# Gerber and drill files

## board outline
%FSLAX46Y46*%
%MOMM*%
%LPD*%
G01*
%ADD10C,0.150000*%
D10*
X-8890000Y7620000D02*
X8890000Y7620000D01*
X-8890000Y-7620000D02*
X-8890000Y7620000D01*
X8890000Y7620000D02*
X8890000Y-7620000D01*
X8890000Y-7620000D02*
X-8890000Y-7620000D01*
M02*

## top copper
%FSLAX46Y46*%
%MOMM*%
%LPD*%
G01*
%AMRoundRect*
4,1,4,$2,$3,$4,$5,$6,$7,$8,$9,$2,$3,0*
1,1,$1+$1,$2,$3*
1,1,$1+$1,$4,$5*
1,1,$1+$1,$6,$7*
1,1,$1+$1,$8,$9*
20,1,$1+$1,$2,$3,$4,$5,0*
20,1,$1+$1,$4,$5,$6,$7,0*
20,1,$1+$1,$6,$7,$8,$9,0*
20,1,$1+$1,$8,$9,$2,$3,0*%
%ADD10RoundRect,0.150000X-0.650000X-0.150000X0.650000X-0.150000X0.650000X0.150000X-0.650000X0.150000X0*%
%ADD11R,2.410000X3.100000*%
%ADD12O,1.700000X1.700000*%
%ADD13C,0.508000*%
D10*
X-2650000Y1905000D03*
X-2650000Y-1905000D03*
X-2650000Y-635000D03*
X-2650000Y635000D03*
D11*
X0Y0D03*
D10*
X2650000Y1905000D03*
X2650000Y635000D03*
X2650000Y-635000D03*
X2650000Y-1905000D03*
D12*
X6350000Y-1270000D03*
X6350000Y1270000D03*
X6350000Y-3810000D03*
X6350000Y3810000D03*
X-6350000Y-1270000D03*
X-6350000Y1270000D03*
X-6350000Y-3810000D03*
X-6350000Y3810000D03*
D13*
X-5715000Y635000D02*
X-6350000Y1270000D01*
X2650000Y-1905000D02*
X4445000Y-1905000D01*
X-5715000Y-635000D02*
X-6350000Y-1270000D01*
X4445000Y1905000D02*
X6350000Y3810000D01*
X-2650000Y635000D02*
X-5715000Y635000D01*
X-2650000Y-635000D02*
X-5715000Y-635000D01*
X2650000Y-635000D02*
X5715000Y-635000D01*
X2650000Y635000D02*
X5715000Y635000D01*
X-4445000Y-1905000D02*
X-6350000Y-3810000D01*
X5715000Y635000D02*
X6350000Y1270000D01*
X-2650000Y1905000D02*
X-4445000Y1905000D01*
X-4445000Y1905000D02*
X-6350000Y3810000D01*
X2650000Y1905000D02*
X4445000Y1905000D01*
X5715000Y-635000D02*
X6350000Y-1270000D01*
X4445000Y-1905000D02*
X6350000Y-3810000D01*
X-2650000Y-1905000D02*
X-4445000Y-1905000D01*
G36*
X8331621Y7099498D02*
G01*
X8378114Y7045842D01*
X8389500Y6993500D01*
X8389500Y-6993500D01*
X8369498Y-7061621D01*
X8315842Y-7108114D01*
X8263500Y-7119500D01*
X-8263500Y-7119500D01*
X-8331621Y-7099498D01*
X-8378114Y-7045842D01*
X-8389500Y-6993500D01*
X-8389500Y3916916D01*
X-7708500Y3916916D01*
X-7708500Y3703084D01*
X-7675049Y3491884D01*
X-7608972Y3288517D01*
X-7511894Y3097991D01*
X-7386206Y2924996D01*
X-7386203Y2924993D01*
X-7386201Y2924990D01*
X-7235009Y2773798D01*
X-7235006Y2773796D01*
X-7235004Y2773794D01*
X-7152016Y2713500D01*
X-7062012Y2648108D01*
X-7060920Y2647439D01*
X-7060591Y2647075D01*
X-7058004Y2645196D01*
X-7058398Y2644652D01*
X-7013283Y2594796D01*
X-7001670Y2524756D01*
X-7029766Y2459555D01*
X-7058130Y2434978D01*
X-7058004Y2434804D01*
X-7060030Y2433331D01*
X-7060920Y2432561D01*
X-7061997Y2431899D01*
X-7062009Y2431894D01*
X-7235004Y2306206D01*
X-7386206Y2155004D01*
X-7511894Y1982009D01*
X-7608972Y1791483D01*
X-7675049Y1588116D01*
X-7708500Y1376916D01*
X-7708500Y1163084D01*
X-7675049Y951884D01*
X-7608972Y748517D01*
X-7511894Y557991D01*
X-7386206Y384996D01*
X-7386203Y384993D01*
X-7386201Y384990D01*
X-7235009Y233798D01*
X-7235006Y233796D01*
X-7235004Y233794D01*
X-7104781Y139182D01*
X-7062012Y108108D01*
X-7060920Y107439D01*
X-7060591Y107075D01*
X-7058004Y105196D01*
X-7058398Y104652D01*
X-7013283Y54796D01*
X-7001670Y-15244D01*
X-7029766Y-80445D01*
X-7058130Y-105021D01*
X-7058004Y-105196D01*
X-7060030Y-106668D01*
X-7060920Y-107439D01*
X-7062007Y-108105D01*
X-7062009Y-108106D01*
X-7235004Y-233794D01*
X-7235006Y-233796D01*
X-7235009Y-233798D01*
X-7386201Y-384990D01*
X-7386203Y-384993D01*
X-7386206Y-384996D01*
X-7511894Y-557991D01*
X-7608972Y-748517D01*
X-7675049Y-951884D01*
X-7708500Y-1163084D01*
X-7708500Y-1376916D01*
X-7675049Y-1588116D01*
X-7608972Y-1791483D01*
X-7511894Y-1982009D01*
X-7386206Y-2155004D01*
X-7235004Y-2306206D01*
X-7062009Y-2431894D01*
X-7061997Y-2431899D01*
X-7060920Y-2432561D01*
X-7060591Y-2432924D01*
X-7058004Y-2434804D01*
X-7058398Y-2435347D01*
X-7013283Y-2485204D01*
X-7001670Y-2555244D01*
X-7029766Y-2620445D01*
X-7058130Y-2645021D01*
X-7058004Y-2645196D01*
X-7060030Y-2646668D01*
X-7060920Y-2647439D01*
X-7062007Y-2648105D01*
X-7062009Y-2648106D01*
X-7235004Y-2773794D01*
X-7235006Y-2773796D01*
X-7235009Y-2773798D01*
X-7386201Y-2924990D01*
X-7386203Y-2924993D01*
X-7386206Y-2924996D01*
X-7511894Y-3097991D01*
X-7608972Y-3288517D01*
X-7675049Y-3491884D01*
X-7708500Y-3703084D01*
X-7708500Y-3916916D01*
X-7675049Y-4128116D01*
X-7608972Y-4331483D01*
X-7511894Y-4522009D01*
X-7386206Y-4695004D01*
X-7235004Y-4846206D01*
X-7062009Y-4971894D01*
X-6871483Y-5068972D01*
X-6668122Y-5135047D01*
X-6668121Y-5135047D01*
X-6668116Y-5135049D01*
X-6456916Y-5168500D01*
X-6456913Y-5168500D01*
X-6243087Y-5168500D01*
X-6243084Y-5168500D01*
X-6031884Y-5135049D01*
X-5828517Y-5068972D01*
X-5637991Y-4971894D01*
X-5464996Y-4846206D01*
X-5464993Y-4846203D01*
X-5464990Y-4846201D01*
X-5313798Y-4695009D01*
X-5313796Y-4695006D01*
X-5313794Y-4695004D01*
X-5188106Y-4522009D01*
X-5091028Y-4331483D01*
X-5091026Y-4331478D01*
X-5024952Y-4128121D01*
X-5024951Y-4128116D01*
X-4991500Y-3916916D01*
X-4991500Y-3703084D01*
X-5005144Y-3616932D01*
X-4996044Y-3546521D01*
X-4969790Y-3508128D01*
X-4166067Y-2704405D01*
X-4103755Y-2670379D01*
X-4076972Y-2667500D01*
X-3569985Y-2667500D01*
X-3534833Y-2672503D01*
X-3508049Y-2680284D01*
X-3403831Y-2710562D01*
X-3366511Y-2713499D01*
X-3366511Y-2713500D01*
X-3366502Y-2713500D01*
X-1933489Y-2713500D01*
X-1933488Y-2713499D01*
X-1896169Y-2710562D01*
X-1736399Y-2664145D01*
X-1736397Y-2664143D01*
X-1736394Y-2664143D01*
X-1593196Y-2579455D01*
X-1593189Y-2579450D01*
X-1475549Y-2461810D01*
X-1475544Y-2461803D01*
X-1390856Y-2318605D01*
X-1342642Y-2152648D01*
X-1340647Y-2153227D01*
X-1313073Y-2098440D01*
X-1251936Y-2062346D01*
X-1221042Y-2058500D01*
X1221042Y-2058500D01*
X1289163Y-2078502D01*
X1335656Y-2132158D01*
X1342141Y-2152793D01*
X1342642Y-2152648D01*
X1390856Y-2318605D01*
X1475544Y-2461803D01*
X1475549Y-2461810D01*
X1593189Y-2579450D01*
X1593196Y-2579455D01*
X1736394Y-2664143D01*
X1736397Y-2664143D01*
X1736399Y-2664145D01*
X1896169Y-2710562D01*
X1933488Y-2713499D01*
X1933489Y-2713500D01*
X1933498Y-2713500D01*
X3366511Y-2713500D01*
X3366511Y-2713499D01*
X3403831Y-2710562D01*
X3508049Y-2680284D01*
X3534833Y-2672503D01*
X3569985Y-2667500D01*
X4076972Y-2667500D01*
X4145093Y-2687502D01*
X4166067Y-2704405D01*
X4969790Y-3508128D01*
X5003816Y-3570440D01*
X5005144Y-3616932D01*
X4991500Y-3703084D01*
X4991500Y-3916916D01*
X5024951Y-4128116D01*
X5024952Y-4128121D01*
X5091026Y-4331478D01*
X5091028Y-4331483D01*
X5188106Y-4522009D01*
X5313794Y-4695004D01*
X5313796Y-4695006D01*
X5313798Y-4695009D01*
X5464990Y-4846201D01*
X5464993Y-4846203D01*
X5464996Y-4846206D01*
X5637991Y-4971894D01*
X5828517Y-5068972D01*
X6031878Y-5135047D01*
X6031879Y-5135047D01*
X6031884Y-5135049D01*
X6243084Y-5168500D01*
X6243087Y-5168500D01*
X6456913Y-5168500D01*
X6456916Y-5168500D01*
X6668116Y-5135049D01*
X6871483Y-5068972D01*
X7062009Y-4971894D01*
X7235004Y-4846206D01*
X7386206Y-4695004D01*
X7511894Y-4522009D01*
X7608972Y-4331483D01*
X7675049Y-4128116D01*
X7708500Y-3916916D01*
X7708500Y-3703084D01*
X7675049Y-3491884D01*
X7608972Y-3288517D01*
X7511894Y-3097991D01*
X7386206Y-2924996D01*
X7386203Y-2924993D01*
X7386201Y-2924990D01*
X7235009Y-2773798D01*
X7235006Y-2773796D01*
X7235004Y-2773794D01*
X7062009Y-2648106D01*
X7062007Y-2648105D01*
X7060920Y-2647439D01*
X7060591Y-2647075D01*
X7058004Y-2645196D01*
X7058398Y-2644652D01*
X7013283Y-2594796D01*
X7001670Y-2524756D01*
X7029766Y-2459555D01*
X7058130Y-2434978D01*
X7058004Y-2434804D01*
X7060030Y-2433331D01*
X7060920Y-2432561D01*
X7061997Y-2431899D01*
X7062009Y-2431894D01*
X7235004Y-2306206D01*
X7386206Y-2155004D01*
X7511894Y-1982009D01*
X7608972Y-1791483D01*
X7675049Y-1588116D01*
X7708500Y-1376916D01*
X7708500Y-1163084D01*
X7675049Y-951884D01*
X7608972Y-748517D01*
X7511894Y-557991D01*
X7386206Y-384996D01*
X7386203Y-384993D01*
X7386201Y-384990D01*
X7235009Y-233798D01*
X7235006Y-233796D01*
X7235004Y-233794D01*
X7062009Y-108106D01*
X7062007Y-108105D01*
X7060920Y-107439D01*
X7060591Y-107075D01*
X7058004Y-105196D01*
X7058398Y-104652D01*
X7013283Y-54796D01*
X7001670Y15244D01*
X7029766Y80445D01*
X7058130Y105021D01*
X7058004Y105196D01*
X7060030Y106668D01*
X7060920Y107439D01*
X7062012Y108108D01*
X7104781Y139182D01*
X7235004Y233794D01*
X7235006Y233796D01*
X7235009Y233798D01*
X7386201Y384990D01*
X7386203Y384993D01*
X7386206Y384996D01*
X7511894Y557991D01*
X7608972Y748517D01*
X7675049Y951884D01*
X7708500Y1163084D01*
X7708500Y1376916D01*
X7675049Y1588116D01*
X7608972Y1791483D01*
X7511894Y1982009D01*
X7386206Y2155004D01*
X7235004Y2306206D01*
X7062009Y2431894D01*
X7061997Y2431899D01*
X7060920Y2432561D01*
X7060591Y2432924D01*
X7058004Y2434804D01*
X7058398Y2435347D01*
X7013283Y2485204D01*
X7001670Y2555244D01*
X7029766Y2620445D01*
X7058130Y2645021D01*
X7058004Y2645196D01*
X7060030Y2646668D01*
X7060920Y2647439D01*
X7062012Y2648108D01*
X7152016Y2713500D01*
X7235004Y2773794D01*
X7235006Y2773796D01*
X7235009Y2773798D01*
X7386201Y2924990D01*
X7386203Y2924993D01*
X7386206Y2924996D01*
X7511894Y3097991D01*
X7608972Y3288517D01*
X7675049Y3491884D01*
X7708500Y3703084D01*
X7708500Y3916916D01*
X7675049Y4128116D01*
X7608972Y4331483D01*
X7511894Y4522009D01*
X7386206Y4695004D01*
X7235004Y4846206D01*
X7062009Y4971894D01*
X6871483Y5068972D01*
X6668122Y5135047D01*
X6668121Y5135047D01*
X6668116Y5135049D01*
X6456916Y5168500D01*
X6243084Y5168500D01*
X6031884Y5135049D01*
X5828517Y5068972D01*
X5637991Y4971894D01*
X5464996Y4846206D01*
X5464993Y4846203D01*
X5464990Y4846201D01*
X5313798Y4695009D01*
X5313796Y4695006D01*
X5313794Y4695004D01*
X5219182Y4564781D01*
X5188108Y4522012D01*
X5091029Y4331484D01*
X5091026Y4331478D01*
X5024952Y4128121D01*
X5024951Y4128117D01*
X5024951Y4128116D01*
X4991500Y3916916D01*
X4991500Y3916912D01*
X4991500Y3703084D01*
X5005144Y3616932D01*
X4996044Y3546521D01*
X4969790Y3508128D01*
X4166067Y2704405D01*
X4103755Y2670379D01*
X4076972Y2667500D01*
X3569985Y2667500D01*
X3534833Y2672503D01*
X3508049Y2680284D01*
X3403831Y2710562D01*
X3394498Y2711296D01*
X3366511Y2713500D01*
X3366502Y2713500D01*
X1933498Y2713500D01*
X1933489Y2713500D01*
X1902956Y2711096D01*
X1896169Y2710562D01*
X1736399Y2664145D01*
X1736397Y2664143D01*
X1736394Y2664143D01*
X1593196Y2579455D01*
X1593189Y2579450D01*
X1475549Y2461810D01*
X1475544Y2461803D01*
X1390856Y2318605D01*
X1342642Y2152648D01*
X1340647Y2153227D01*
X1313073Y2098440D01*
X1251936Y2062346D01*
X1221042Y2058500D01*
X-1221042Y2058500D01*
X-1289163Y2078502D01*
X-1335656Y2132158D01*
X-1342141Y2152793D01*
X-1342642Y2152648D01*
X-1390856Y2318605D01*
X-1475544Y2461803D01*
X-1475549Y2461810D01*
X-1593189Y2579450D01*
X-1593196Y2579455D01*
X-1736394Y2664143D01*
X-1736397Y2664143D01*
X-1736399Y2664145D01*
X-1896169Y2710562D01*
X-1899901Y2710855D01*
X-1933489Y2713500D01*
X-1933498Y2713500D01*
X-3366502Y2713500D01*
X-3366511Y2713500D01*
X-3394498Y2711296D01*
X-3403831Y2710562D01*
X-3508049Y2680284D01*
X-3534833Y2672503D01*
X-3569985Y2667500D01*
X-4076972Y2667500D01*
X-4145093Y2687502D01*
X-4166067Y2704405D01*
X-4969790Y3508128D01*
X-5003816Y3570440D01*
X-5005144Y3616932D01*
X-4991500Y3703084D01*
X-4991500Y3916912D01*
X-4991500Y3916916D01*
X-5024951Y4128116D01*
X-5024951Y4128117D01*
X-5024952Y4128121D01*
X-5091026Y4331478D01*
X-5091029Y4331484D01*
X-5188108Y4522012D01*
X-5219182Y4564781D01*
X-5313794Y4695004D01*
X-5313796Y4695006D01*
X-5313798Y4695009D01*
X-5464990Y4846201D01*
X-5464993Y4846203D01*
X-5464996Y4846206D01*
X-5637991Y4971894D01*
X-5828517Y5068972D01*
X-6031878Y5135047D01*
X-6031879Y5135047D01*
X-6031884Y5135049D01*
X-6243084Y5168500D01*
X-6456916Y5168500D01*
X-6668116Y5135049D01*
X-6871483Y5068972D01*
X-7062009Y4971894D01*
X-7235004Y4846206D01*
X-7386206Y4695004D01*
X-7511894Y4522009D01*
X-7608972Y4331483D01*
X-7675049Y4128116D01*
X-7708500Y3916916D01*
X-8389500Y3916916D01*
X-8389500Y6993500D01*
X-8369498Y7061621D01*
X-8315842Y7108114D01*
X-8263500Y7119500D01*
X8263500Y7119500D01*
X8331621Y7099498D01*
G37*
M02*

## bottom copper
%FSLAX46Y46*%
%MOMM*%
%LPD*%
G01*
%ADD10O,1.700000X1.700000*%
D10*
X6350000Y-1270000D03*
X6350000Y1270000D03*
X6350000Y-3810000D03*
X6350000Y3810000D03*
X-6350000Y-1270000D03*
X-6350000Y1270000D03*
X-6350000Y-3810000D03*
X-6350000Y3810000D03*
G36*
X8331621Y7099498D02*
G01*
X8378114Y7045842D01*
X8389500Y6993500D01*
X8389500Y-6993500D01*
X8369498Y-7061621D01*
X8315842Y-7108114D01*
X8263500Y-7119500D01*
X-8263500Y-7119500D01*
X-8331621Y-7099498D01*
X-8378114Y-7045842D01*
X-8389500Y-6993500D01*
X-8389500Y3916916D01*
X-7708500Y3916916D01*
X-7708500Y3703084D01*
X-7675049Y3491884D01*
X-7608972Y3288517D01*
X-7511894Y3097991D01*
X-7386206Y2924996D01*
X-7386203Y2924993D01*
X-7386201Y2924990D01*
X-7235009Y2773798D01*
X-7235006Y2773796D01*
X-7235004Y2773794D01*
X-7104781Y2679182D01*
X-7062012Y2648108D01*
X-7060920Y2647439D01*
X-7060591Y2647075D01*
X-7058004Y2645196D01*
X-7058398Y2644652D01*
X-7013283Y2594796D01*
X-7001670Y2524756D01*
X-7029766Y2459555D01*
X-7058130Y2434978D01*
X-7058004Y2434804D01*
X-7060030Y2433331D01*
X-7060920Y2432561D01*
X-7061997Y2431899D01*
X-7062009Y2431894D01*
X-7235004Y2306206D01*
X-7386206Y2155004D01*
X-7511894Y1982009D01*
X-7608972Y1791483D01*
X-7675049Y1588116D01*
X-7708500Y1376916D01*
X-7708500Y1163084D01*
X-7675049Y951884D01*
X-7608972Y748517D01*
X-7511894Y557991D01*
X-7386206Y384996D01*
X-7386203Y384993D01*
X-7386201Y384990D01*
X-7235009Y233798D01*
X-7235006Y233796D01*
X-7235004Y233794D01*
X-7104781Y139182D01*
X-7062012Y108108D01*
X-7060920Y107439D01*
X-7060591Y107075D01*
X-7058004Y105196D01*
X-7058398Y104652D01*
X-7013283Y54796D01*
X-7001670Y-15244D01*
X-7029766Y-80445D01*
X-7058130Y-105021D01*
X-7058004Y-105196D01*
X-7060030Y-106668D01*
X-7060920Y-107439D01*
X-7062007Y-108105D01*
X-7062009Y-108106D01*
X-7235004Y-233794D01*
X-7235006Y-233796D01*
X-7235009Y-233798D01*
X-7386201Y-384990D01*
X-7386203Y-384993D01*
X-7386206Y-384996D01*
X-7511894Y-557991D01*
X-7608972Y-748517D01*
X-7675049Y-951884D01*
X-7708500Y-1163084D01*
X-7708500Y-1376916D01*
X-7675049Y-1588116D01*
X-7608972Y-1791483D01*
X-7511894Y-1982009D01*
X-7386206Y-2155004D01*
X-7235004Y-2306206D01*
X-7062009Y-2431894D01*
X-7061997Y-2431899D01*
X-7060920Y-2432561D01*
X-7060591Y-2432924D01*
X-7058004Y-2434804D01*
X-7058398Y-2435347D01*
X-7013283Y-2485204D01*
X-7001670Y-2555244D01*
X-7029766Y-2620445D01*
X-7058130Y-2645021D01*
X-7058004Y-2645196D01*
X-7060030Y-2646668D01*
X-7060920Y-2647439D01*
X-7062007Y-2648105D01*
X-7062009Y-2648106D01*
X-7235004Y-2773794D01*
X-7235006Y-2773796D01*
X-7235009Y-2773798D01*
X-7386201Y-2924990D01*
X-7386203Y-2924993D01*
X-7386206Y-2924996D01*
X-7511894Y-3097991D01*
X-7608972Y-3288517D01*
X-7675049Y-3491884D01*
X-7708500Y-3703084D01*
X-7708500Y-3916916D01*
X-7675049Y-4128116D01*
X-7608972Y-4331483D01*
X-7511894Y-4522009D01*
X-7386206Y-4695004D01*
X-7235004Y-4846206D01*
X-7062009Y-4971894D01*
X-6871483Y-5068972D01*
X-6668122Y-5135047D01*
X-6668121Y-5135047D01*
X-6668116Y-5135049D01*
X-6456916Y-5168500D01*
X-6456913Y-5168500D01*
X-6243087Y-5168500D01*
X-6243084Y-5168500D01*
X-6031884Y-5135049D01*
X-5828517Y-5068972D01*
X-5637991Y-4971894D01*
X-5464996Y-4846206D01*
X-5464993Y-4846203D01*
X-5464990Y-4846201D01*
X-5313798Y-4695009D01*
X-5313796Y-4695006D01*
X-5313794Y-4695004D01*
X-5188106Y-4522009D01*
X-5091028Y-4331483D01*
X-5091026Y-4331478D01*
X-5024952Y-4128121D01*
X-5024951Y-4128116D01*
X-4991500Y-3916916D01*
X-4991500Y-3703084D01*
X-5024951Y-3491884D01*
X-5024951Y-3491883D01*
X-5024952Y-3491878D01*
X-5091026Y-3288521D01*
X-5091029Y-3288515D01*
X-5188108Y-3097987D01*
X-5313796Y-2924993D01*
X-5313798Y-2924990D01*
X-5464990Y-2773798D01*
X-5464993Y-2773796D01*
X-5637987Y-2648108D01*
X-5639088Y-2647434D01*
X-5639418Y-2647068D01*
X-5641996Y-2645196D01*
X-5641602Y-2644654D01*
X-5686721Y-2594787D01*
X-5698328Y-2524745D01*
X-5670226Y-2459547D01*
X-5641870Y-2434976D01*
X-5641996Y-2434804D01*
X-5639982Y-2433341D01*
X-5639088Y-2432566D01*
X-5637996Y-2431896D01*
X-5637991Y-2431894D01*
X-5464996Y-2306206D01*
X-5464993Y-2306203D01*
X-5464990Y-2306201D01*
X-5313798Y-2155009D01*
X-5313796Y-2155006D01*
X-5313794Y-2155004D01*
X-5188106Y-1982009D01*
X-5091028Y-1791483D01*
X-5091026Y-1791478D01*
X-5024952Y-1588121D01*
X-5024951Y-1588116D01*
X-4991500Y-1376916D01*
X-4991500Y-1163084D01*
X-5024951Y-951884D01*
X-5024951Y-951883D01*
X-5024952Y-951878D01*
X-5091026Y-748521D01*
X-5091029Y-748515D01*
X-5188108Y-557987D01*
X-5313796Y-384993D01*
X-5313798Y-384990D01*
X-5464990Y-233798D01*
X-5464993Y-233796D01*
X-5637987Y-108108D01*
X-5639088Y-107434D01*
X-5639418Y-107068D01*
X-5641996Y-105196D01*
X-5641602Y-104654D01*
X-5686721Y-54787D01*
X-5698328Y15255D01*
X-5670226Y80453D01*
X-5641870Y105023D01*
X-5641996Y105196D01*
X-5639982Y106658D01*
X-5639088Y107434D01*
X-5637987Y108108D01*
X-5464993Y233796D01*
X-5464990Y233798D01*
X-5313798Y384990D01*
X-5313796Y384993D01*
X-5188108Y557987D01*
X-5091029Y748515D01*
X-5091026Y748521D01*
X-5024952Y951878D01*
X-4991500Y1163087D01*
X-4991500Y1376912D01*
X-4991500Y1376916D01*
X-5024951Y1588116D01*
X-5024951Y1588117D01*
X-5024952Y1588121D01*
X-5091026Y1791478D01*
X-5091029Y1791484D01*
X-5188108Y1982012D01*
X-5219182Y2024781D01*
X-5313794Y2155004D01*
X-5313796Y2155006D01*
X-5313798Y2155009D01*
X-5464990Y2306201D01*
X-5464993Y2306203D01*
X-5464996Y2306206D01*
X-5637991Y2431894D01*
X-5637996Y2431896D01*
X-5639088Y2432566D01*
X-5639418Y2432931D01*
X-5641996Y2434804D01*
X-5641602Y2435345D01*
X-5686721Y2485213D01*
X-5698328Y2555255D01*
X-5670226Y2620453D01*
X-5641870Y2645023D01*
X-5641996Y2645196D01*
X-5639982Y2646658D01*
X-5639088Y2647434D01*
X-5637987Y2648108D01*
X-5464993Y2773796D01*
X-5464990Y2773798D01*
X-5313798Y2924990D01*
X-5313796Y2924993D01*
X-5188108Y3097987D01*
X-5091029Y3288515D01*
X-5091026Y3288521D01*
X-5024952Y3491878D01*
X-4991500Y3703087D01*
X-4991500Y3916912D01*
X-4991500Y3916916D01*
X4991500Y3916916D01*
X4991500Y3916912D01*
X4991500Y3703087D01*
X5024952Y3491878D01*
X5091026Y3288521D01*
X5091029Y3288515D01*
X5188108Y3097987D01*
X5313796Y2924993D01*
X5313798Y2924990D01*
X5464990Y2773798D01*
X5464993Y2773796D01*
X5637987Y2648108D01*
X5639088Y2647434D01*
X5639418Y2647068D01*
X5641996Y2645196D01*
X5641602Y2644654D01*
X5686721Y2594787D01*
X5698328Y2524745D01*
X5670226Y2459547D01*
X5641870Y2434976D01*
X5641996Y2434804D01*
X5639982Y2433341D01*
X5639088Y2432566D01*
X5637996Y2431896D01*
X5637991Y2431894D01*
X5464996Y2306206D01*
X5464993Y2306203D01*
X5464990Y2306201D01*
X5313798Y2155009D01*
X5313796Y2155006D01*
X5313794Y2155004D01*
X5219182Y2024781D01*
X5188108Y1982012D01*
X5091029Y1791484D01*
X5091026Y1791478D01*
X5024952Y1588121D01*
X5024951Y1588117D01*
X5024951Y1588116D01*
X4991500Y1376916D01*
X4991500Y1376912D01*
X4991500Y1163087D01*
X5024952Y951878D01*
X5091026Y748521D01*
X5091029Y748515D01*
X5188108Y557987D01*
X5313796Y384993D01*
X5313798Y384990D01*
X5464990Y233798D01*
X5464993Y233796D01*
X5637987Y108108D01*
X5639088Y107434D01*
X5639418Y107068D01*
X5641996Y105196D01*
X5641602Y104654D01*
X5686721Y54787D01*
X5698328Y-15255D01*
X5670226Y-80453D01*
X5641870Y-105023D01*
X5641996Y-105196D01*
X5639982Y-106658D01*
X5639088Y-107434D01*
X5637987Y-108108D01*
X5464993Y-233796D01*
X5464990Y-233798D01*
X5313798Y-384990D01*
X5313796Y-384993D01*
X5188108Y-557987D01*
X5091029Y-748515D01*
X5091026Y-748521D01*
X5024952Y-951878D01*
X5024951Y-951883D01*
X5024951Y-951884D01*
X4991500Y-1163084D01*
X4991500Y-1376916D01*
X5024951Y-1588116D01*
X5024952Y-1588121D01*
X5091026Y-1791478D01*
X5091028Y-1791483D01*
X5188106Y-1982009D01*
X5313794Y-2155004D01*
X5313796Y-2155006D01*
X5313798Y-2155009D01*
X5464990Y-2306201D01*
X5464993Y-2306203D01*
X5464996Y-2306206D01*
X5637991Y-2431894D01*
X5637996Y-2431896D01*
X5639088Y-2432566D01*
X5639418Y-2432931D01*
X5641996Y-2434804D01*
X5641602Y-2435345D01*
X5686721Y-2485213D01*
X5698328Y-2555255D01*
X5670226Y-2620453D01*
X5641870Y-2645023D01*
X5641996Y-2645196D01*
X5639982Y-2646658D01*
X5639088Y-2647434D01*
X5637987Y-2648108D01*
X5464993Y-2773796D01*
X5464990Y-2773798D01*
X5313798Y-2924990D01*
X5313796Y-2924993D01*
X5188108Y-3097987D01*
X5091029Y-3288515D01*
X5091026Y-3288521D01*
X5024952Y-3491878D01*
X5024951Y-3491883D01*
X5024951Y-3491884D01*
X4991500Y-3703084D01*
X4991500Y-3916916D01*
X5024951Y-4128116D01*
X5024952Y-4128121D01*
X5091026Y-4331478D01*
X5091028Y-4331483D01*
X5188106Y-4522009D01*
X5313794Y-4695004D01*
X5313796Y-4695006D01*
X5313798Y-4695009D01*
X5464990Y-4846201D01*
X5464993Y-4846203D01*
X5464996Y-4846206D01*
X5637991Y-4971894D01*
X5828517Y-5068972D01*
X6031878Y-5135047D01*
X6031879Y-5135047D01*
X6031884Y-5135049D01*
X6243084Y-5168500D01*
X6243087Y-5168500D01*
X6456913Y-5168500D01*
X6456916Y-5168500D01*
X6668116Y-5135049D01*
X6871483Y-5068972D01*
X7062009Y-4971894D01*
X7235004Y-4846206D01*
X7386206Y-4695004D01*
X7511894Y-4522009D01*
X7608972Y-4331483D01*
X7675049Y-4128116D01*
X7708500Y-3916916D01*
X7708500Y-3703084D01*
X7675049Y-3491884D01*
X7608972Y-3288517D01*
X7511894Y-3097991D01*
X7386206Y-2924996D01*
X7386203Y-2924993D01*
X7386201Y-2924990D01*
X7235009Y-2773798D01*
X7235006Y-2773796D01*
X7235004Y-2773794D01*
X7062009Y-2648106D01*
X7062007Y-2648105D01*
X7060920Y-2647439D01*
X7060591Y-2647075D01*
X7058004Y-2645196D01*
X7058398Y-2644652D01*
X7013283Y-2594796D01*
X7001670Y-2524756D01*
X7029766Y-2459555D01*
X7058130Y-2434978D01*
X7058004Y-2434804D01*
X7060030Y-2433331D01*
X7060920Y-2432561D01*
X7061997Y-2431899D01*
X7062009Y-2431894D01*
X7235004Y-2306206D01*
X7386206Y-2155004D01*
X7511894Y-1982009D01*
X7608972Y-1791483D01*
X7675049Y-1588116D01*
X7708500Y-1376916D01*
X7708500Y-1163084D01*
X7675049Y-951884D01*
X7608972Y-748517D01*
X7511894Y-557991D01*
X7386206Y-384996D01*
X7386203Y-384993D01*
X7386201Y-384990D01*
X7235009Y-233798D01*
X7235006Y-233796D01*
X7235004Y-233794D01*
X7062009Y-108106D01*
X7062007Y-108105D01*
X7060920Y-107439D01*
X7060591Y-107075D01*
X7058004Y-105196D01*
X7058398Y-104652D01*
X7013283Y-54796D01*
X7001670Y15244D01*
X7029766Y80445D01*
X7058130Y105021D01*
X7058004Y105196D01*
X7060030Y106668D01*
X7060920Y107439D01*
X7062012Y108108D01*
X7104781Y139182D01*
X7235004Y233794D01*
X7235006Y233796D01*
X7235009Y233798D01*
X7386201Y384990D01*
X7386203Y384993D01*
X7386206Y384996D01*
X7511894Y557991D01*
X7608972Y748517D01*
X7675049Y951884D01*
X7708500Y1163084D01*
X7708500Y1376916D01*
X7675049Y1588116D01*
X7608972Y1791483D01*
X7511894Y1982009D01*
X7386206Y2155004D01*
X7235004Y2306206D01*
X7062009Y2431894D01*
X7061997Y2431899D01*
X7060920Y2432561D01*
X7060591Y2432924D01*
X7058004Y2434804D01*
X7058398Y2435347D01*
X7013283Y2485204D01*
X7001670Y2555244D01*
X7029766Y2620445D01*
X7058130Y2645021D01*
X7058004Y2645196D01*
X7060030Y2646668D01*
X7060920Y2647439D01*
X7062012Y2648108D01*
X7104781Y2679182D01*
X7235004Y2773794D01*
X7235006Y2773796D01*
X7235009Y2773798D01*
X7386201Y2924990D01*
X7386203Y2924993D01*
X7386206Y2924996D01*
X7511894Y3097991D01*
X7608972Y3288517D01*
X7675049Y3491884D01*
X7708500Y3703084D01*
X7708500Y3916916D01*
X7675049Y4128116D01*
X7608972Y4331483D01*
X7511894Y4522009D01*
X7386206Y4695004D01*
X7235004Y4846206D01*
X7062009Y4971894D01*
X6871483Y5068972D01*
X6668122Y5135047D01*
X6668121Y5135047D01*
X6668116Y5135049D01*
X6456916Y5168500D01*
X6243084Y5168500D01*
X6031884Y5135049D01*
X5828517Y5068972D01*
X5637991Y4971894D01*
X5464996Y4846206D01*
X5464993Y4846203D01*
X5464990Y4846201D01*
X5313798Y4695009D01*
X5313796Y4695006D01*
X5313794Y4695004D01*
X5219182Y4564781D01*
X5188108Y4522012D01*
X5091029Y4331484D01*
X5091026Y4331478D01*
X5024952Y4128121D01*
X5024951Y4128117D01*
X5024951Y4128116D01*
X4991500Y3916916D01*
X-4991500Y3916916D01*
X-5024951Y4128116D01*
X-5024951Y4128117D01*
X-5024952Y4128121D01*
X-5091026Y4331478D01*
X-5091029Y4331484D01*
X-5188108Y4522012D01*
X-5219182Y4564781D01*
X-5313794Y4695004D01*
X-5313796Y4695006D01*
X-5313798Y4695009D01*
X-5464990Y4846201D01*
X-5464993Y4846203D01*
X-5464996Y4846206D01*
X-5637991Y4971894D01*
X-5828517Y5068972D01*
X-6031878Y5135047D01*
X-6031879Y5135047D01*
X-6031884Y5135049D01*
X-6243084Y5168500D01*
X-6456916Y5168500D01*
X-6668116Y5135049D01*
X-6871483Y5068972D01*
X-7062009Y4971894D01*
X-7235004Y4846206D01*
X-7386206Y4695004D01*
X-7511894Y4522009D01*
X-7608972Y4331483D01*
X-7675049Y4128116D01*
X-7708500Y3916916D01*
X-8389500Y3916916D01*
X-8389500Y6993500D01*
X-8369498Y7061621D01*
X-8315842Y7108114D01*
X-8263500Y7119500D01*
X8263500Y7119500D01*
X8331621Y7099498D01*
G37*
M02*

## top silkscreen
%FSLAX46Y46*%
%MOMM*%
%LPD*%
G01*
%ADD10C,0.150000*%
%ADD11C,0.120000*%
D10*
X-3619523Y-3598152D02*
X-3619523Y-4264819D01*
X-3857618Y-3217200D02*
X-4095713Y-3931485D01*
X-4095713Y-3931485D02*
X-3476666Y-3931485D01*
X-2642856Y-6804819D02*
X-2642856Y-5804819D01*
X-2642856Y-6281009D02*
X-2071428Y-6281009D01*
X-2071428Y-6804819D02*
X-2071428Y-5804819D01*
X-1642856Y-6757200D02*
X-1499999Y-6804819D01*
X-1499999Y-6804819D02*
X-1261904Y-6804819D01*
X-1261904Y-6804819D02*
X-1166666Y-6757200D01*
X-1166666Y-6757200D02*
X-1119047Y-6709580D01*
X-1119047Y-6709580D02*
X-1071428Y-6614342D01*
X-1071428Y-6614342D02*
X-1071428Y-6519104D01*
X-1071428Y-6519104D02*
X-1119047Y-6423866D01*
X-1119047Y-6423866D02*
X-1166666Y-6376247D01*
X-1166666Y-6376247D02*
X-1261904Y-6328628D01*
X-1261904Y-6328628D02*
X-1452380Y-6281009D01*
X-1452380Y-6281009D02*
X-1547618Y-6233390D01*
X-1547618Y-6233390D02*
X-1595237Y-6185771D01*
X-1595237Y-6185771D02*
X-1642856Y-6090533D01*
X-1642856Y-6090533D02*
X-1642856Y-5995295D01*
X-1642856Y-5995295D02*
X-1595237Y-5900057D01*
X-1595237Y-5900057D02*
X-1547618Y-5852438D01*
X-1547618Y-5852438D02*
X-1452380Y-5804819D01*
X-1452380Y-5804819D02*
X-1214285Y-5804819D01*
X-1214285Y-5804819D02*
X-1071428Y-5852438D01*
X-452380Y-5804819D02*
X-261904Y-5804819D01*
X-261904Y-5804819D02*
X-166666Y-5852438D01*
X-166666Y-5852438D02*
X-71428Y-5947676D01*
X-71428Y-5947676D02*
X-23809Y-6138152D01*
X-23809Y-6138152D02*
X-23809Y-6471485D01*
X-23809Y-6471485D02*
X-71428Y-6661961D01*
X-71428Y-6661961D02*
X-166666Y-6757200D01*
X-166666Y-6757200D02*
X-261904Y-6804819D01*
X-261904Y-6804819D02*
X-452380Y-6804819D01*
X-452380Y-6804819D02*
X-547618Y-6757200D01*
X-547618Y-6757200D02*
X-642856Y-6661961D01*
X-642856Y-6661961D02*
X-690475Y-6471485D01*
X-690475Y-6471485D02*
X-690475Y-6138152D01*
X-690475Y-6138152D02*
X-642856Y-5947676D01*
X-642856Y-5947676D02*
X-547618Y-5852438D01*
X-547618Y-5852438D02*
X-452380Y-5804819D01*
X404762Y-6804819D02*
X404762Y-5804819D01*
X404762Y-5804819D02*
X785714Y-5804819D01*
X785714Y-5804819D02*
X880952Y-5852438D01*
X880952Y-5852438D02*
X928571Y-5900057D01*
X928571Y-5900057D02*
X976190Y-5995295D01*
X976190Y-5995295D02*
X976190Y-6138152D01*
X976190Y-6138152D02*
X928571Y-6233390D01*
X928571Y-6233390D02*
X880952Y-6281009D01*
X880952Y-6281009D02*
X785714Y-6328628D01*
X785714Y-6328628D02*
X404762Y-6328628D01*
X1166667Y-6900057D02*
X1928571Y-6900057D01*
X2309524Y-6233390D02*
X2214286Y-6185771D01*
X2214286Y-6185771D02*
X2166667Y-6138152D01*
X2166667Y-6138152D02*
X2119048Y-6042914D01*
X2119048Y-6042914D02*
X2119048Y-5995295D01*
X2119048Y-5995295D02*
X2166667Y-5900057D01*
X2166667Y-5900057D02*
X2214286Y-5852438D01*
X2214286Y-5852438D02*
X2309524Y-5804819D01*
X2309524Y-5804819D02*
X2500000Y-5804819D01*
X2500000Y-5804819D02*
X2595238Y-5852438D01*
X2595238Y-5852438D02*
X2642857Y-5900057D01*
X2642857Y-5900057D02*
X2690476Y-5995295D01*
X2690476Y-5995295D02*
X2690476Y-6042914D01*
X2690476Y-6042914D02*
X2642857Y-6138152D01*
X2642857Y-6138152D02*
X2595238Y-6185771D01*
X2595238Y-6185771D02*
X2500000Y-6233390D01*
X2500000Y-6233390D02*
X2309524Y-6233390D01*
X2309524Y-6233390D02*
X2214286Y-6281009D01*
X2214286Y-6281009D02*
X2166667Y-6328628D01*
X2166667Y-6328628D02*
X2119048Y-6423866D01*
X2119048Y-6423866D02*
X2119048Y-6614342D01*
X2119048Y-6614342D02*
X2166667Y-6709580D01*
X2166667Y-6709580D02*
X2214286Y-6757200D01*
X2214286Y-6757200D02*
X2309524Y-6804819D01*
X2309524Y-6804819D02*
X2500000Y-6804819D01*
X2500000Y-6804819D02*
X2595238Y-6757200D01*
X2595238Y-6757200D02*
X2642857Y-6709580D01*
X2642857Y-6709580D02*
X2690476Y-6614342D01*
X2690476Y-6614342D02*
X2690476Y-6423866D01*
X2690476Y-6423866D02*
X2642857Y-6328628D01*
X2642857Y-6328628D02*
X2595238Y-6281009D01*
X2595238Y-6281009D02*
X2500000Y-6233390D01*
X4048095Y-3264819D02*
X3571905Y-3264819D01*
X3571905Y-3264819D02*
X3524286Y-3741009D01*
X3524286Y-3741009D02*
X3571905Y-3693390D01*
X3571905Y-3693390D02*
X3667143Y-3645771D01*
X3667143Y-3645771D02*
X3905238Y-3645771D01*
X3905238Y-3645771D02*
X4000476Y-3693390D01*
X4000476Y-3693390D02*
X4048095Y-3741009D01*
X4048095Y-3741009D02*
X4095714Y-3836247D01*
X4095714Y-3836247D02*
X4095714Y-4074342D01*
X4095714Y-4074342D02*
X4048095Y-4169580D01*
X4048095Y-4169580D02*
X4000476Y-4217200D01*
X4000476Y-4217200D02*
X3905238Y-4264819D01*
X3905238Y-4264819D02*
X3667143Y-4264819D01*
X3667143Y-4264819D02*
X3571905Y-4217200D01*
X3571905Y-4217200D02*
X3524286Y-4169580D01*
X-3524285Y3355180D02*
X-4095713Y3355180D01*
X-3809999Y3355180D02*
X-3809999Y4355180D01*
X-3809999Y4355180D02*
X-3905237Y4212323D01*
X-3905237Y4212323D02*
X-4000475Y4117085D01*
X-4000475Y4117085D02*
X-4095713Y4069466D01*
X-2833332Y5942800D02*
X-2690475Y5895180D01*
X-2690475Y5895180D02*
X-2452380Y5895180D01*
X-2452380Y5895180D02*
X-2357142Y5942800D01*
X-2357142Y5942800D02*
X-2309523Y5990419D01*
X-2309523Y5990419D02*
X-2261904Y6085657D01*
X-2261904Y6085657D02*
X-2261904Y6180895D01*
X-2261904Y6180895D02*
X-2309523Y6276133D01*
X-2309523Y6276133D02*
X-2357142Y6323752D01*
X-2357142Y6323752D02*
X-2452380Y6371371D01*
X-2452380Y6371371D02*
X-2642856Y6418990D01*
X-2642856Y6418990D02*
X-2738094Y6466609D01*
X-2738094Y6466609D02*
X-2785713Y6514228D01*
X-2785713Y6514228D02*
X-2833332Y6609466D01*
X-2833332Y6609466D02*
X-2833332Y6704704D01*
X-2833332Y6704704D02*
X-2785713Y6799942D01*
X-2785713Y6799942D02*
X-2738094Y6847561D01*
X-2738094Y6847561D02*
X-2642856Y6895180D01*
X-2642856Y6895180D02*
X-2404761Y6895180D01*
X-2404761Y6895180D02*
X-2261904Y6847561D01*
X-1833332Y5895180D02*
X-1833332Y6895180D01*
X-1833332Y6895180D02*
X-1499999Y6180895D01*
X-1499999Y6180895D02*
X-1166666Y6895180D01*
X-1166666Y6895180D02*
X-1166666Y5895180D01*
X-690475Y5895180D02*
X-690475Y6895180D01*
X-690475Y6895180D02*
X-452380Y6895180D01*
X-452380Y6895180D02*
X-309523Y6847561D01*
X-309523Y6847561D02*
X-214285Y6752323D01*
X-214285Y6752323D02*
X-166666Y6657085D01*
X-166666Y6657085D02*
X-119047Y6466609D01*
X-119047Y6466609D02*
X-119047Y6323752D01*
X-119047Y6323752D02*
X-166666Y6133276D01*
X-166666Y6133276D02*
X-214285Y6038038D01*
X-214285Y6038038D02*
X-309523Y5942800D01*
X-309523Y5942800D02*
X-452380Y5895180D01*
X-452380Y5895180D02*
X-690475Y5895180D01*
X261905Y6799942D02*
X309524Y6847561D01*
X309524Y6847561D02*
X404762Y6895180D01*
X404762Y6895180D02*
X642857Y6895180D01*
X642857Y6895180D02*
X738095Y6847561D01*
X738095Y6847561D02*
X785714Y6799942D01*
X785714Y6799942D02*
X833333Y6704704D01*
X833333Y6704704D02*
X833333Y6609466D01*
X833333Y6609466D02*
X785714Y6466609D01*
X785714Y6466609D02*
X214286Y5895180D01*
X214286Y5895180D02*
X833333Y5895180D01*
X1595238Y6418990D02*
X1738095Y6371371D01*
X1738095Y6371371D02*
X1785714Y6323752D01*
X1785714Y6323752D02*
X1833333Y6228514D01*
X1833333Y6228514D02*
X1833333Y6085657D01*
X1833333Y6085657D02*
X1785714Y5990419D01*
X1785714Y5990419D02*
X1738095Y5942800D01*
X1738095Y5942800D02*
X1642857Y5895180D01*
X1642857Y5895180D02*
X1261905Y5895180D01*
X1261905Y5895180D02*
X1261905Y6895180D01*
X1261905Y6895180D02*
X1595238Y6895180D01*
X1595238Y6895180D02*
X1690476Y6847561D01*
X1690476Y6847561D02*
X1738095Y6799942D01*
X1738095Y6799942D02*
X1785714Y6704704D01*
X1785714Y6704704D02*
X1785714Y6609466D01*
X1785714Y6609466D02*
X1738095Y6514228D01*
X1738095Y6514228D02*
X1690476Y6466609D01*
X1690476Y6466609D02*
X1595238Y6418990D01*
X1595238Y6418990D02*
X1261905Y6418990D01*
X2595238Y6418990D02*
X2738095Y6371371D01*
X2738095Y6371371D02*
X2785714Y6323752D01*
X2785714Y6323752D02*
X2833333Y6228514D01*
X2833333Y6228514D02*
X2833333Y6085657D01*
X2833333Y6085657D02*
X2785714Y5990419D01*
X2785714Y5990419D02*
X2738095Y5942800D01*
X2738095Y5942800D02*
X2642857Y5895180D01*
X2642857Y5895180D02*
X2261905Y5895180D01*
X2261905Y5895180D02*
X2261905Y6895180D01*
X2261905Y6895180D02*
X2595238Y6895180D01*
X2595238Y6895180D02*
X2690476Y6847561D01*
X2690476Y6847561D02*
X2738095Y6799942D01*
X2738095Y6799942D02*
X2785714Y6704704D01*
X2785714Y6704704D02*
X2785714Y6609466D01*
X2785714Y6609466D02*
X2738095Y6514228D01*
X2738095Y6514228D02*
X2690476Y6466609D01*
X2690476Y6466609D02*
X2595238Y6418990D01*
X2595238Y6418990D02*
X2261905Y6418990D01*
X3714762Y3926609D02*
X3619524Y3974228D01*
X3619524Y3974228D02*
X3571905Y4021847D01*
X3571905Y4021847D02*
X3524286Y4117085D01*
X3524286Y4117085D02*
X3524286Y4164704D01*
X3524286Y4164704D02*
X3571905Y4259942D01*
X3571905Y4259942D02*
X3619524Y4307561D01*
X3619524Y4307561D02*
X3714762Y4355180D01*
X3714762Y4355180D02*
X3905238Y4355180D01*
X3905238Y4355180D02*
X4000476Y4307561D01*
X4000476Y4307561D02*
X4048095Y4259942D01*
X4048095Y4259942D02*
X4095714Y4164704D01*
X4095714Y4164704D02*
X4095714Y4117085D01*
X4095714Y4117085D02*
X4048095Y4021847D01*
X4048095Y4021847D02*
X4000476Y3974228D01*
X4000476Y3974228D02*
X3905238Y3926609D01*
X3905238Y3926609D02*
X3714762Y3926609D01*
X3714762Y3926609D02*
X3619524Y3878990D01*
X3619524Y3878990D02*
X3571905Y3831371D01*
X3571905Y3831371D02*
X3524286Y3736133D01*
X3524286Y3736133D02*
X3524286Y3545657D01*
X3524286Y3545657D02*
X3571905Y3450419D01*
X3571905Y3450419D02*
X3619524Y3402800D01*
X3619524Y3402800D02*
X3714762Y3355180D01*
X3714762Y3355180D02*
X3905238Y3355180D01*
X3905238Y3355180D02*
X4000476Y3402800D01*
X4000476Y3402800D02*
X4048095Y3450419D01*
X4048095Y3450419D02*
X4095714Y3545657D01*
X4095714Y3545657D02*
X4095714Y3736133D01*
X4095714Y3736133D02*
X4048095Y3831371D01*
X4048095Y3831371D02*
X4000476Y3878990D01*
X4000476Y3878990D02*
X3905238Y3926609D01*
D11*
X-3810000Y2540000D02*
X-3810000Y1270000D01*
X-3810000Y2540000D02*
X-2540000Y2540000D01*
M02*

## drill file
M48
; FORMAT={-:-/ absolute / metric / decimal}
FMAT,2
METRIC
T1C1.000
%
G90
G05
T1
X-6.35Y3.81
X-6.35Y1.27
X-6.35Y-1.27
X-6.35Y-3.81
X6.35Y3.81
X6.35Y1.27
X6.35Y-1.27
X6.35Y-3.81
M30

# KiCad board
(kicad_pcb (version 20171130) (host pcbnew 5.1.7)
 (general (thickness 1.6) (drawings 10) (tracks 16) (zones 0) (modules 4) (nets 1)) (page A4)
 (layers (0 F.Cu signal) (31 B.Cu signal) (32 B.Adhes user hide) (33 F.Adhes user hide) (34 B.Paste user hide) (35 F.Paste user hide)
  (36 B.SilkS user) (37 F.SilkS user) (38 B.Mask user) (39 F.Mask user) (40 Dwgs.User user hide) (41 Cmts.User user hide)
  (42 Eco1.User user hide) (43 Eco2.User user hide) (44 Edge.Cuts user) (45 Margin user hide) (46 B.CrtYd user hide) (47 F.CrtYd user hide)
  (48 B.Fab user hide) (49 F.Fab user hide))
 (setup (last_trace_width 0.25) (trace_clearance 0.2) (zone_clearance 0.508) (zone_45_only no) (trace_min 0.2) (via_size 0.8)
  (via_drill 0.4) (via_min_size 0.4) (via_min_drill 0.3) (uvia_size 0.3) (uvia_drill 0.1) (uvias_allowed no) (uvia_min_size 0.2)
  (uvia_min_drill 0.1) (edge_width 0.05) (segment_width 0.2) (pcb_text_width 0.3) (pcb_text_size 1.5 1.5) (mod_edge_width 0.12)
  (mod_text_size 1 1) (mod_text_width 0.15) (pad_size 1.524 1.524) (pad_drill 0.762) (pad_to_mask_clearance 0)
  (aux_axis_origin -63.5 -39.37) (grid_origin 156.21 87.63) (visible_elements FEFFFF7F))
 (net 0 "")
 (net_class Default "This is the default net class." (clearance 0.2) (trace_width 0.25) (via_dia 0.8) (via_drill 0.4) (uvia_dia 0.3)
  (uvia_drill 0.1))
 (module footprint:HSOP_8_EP (layer F.Cu) (at 0 0)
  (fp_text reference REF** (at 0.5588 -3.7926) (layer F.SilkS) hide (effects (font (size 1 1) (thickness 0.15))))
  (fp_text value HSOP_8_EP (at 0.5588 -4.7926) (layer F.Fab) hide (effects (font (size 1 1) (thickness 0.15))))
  (fp_line (start -3.81 -2.54) (end -3.81 -1.27) (layer F.SilkS) (width 0.12))
  (fp_line (start -3.81 -2.54) (end -2.54 -2.54) (layer F.SilkS) (width 0.12))
  (pad 1 smd roundrect (at -2.65 -1.905) (size 1.6 0.6) (layers F.Cu F.Paste F.Mask) (roundrect_rratio 0.25))
  (pad 4 smd roundrect (at -2.65 1.905) (size 1.6 0.6) (layers F.Cu F.Paste F.Mask) (roundrect_rratio 0.25))
  (pad 3 smd roundrect (at -2.65 0.635) (size 1.6 0.6) (layers F.Cu F.Paste F.Mask) (roundrect_rratio 0.25))
  (pad 2 smd roundrect (at -2.65 -0.635) (size 1.6 0.6) (layers F.Cu F.Paste F.Mask) (roundrect_rratio 0.25))
  (pad "" smd roundrect (at -0.6 0.775) (size 0.97 1.25) (layers F.Paste) (roundrect_rratio 0.25))
  (pad 9 smd rect (at 0 0) (size 2.41 3.1) (layers F.Cu F.Mask))
  (pad 8 smd roundrect (at 2.65 -1.905) (size 1.6 0.6) (layers F.Cu F.Paste F.Mask) (roundrect_rratio 0.25))
  (pad 7 smd roundrect (at 2.65 -0.635) (size 1.6 0.6) (layers F.Cu F.Paste F.Mask) (roundrect_rratio 0.25))
  (pad "" smd roundrect (at 0.6 0.775) (size 0.97 1.25) (layers F.Paste) (roundrect_rratio 0.25))
  (pad 6 smd roundrect (at 2.65 0.635) (size 1.6 0.6) (layers F.Cu F.Paste F.Mask) (roundrect_rratio 0.25))
  (pad 5 smd roundrect (at 2.65 1.905) (size 1.6 0.6) (layers F.Cu F.Paste F.Mask) (roundrect_rratio 0.25))
  (pad "" smd roundrect (at 0.6 -0.775) (size 0.97 1.25) (layers F.Paste) (roundrect_rratio 0.25))
  (pad "" smd roundrect (at -0.6 -0.775) (size 0.97 1.25) (layers F.Paste) (roundrect_rratio 0.25)))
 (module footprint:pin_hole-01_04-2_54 (layer F.Cu) (at 6.35 0)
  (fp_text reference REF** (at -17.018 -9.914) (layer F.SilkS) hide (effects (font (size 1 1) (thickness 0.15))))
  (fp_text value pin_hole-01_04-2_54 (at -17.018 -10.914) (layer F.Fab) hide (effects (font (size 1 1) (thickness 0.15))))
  (pad 3 thru_hole oval (at 0 1.27) (size 1.7 1.7) (drill 1) (layers *.Cu *.Mask))
  (pad 2 thru_hole oval (at 0 -1.27) (size 1.7 1.7) (drill 1) (layers *.Cu *.Mask))
  (pad 4 thru_hole oval (at 0 3.81) (size 1.7 1.7) (drill 1) (layers *.Cu *.Mask))
  (pad 1 thru_hole oval (at 0 -3.81) (size 1.7 1.7) (drill 1) (layers *.Cu *.Mask)))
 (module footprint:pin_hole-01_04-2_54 (layer F.Cu) (at -6.35 0)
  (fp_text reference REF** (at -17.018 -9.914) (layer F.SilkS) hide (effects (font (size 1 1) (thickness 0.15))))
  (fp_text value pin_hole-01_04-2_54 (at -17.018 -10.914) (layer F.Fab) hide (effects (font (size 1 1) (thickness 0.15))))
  (pad 3 thru_hole oval (at 0 1.27) (size 1.7 1.7) (drill 1) (layers *.Cu *.Mask))
  (pad 2 thru_hole oval (at 0 -1.27) (size 1.7 1.7) (drill 1) (layers *.Cu *.Mask))
  (pad 4 thru_hole oval (at 0 3.81) (size 1.7 1.7) (drill 1) (layers *.Cu *.Mask))
  (pad 1 thru_hole oval (at 0 -3.81) (size 1.7 1.7) (drill 1) (layers *.Cu *.Mask)))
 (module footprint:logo (layer B.Cu) (at 0 0 180)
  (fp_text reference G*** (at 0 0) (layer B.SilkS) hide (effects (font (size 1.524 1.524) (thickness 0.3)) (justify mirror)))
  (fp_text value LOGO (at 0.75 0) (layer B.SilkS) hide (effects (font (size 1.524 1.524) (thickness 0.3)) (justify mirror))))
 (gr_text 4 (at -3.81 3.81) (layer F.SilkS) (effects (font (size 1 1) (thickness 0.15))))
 (gr_line (start -8.89 -7.62) (end 8.89 -7.62) (layer Edge.Cuts) (width 0.15))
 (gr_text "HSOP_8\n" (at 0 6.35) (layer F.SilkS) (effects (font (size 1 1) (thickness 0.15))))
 (gr_line (start -8.89 7.62) (end -8.89 -7.62) (layer Edge.Cuts) (width 0.15))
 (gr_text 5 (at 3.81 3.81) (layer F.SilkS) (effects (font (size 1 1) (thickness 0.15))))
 (gr_line (start 8.89 -7.62) (end 8.89 7.62) (layer Edge.Cuts) (width 0.15))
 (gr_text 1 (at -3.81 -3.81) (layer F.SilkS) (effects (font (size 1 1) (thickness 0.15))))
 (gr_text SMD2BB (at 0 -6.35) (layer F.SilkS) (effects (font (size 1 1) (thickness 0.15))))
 (gr_line (start 8.89 7.62) (end -8.89 7.62) (layer Edge.Cuts) (width 0.15))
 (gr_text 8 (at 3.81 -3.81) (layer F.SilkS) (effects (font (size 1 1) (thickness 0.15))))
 (segment (start -5.715 -0.635) (end -6.35 -1.27) (width 0.508) (layer F.Cu) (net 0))
 (segment (start 2.65 1.905) (end 4.445 1.905) (width 0.508) (layer F.Cu) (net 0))
 (segment (start -5.715 0.635) (end -6.35 1.27) (width 0.508) (layer F.Cu) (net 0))
 (segment (start 4.445 -1.905) (end 6.35 -3.81) (width 0.508) (layer F.Cu) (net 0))
 (segment (start -2.65 -0.635) (end -5.715 -0.635) (width 0.508) (layer F.Cu) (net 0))
 (segment (start -2.65 0.635) (end -5.715 0.635) (width 0.508) (layer F.Cu) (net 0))
 (segment (start 2.65 0.635) (end 5.715 0.635) (width 0.508) (layer F.Cu) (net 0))
 (segment (start 2.65 -0.635) (end 5.715 -0.635) (width 0.508) (layer F.Cu) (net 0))
 (segment (start -4.445 1.905) (end -6.35 3.81) (width 0.508) (layer F.Cu) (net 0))
 (segment (start 5.715 -0.635) (end 6.35 -1.27) (width 0.508) (layer F.Cu) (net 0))
 (segment (start -2.65 -1.905) (end -4.445 -1.905) (width 0.508) (layer F.Cu) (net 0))
 (segment (start -4.445 -1.905) (end -6.35 -3.81) (width 0.508) (layer F.Cu) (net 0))
 (segment (start 2.65 -1.905) (end 4.445 -1.905) (width 0.508) (layer F.Cu) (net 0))
 (segment (start 5.715 0.635) (end 6.35 1.27) (width 0.508) (layer F.Cu) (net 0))
 (segment (start 4.445 1.905) (end 6.35 3.81) (width 0.508) (layer F.Cu) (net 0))
 (segment (start -2.65 1.905) (end -4.445 1.905) (width 0.508) (layer F.Cu) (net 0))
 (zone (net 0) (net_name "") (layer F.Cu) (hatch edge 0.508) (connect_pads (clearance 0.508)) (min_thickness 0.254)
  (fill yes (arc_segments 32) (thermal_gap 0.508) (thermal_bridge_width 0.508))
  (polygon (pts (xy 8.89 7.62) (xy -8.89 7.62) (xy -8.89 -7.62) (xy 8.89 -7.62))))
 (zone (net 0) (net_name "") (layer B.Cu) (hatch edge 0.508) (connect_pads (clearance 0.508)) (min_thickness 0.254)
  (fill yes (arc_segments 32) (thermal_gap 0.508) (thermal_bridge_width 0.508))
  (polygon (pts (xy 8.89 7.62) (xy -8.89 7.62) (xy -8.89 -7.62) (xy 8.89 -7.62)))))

